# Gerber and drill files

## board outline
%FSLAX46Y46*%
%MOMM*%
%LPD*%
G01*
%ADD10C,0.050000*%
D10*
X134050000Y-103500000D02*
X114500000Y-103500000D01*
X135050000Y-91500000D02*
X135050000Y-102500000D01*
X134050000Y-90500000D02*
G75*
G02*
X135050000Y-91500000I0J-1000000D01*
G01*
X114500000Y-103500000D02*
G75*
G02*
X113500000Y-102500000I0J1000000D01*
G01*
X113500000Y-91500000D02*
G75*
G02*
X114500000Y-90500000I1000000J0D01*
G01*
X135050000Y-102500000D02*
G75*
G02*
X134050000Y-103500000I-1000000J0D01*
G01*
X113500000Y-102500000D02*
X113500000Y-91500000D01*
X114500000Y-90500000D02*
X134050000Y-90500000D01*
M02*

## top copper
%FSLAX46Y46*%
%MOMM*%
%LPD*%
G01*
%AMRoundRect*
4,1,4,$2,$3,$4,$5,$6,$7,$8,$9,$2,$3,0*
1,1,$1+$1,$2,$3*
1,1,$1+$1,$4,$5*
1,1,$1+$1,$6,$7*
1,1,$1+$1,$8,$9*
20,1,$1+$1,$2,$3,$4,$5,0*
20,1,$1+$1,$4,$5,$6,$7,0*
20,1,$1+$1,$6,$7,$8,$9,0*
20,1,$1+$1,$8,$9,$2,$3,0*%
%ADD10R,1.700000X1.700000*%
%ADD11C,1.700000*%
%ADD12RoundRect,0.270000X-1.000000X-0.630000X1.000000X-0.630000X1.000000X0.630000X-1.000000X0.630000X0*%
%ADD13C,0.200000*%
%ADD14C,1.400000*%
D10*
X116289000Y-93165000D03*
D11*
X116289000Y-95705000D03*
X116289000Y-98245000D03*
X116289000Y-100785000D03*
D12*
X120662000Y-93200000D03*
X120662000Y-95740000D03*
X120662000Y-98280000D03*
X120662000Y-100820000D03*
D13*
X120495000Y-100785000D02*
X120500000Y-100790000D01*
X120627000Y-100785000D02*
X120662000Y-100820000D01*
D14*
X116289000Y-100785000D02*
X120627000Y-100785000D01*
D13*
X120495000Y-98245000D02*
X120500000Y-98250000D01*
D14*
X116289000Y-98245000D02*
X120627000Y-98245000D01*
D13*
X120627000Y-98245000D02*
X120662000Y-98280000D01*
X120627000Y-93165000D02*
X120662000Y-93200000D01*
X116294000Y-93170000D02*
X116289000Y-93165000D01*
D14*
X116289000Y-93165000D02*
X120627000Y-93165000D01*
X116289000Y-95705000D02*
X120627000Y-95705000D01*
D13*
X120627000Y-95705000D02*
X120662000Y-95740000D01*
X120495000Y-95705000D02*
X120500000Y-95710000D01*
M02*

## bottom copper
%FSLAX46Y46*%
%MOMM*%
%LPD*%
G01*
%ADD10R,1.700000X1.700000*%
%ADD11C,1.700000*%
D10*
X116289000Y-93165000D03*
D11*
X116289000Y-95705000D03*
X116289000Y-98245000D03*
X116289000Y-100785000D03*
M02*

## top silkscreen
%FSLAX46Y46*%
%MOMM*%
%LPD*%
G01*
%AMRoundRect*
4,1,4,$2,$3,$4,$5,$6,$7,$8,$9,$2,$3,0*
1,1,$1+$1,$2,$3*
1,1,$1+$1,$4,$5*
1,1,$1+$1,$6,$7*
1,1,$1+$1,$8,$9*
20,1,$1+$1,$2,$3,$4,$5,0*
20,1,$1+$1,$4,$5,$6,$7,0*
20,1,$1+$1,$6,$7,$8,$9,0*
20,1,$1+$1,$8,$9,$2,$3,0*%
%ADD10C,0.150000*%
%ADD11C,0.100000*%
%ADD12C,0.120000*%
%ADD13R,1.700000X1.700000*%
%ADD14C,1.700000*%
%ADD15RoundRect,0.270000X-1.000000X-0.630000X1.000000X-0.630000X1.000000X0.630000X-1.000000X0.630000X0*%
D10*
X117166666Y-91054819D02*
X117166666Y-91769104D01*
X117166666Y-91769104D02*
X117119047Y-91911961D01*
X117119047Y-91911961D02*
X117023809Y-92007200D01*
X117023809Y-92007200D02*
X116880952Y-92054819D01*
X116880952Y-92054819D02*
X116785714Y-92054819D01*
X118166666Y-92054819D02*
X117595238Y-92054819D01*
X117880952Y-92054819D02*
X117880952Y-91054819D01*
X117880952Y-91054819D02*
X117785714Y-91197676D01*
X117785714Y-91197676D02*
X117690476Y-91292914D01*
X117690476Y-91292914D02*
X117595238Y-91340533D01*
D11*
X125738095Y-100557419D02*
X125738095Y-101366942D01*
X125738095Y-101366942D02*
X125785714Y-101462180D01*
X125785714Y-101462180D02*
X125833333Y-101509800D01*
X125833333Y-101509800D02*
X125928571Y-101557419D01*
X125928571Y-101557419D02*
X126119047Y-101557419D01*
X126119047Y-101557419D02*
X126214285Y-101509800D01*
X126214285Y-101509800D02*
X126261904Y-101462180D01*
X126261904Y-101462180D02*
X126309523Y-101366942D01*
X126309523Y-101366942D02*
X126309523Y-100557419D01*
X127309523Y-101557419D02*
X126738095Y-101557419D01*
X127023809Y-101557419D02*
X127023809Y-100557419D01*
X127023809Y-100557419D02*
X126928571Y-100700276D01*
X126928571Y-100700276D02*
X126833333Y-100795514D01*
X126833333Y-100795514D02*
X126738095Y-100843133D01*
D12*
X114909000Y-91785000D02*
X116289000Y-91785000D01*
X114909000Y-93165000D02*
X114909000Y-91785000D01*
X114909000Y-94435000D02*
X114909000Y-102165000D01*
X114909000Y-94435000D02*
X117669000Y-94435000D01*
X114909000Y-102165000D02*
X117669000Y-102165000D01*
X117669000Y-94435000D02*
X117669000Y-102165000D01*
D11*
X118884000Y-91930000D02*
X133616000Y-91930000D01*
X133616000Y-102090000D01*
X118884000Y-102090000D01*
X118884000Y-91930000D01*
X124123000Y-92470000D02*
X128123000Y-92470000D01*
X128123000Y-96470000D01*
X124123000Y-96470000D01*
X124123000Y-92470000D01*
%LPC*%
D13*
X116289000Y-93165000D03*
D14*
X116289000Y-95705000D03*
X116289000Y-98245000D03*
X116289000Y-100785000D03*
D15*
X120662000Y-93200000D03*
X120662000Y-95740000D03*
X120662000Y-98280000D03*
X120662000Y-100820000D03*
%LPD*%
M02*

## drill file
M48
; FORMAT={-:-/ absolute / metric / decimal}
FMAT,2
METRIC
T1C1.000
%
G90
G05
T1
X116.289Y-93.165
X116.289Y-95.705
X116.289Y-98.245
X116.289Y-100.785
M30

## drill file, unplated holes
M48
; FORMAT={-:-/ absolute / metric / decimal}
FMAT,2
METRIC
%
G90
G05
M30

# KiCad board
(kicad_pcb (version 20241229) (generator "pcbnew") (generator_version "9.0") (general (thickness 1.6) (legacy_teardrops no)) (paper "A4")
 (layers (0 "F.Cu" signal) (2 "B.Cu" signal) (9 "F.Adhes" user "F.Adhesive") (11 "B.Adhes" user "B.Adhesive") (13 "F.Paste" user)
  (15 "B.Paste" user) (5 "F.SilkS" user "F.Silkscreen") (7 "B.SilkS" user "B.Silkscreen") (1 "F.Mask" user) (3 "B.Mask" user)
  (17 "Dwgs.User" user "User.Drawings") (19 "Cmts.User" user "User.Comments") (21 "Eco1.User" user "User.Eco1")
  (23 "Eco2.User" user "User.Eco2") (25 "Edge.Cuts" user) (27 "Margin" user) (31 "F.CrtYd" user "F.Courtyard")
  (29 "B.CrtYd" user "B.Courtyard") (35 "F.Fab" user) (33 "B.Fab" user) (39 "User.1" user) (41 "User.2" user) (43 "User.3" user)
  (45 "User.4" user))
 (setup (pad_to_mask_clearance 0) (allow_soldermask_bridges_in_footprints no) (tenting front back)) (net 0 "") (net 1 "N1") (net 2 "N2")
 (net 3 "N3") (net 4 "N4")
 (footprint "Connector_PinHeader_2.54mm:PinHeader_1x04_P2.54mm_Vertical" (layer "F.Cu") (at 116.289 93.165)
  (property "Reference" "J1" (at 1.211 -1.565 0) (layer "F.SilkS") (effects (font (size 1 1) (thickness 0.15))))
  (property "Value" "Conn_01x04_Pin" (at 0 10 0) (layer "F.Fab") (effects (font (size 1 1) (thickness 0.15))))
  (fp_line (start -1.38 -1.38) (end 0 -1.38) (stroke (width 0.12) (type solid)) (layer "F.SilkS"))
  (fp_line (start -1.38 0) (end -1.38 -1.38) (stroke (width 0.12) (type solid)) (layer "F.SilkS"))
  (fp_line (start -1.38 1.27) (end -1.38 9) (stroke (width 0.12) (type solid)) (layer "F.SilkS"))
  (fp_line (start -1.38 1.27) (end 1.38 1.27) (stroke (width 0.12) (type solid)) (layer "F.SilkS"))
  (fp_line (start -1.38 9) (end 1.38 9) (stroke (width 0.12) (type solid)) (layer "F.SilkS"))
  (fp_line (start 1.38 1.27) (end 1.38 9) (stroke (width 0.12) (type solid)) (layer "F.SilkS"))
  (pad "1" thru_hole rect (at 0 0) (size 1.7 1.7) (drill 1) (layers "*.Cu" "*.Mask") (remove_unused_layers no) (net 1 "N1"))
  (pad "2" thru_hole circle (at 0 2.54) (size 1.7 1.7) (drill 1) (layers "*.Cu" "*.Mask") (remove_unused_layers no) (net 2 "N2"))
  (pad "3" thru_hole circle (at 0 5.08) (size 1.7 1.7) (drill 1) (layers "*.Cu" "*.Mask") (remove_unused_layers no) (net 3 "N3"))
  (pad "4" thru_hole circle (at 0 7.62) (size 1.7 1.7) (drill 1) (layers "*.Cu" "*.Mask") (remove_unused_layers no) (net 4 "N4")))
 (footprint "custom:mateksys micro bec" (layer "F.Cu") (at 126.25 97.01)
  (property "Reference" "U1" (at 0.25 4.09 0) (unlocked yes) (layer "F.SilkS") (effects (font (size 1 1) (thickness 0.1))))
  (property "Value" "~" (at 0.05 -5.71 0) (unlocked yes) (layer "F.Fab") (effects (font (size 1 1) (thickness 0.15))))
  (fp_rect (start -7.366 -5.08) (end 7.366 5.08) (stroke (width 0.1) (type default)) (fill no) (layer "F.SilkS"))
  (fp_rect (start -2.127 -4.54) (end 1.873 -0.54) (stroke (width 0.1) (type solid)) (fill no) (layer "F.SilkS"))
  (pad "1" smd roundrect (at -5.588 -3.81) (size 2.54 1.8) (layers "F.Cu" "F.Mask" "F.Paste") (roundrect_rratio 0.15) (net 1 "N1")
   (thermal_bridge_angle 45))
  (pad "2" smd roundrect (at -5.588 -1.27) (size 2.54 1.8) (layers "F.Cu" "F.Mask" "F.Paste") (roundrect_rratio 0.15) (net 2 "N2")
   (thermal_bridge_angle 45))
  (pad "3" smd roundrect (at -5.588 1.27) (size 2.54 1.8) (layers "F.Cu" "F.Mask" "F.Paste") (roundrect_rratio 0.15) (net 3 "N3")
   (thermal_bridge_angle 45))
  (pad "4" smd roundrect (at -5.588 3.81) (size 2.54 1.8) (layers "F.Cu" "F.Mask" "F.Paste") (roundrect_rratio 0.15) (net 4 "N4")
   (thermal_bridge_angle 45)))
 (gr_line (start 134.05 103.5) (end 114.5 103.5) (stroke (width 0.05) (type default)) (layer "Edge.Cuts"))
 (gr_line (start 135.05 91.5) (end 135.05 102.5) (stroke (width 0.05) (type default)) (layer "Edge.Cuts"))
 (gr_arc (start 134.05 90.5) (mid 134.757107 90.792893) (end 135.05 91.5) (stroke (width 0.05) (type default)) (layer "Edge.Cuts"))
 (gr_arc (start 114.5 103.5) (mid 113.792893 103.207107) (end 113.5 102.5) (stroke (width 0.05) (type default)) (layer "Edge.Cuts"))
 (gr_arc (start 113.5 91.5) (mid 113.792893 90.792893) (end 114.5 90.5) (stroke (width 0.05) (type default)) (layer "Edge.Cuts"))
 (gr_arc (start 135.05 102.5) (mid 134.757107 103.207107) (end 134.05 103.5) (stroke (width 0.05) (type default)) (layer "Edge.Cuts"))
 (gr_line (start 113.5 102.5) (end 113.5 91.5) (stroke (width 0.05) (type default)) (layer "Edge.Cuts"))
 (gr_line (start 114.5 90.5) (end 134.05 90.5) (stroke (width 0.05) (type default)) (layer "Edge.Cuts"))
 (segment (start 120.495 100.785) (end 120.5 100.79) (width 0.2) (layer "F.Cu") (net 4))
 (segment (start 120.627 100.785) (end 120.662 100.82) (width 0.2) (layer "F.Cu") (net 4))
 (segment (start 116.289 100.785) (end 120.627 100.785) (width 1.4) (layer "F.Cu") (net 4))
 (segment (start 120.495 98.245) (end 120.5 98.25) (width 0.2) (layer "F.Cu") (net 3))
 (segment (start 116.289 98.245) (end 120.627 98.245) (width 1.4) (layer "F.Cu") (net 3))
 (segment (start 120.627 98.245) (end 120.662 98.28) (width 0.2) (layer "F.Cu") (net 3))
 (segment (start 120.627 93.165) (end 120.662 93.2) (width 0.2) (layer "F.Cu") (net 1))
 (segment (start 116.294 93.17) (end 116.289 93.165) (width 0.2) (layer "F.Cu") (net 1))
 (segment (start 116.289 93.165) (end 120.627 93.165) (width 1.4) (layer "F.Cu") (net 1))
 (segment (start 116.289 95.705) (end 120.627 95.705) (width 1.4) (layer "F.Cu") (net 2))
 (segment (start 120.627 95.705) (end 120.662 95.74) (width 0.2) (layer "F.Cu") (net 2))
 (segment (start 120.495 95.705) (end 120.5 95.71) (width 0.2) (layer "F.Cu") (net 2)))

